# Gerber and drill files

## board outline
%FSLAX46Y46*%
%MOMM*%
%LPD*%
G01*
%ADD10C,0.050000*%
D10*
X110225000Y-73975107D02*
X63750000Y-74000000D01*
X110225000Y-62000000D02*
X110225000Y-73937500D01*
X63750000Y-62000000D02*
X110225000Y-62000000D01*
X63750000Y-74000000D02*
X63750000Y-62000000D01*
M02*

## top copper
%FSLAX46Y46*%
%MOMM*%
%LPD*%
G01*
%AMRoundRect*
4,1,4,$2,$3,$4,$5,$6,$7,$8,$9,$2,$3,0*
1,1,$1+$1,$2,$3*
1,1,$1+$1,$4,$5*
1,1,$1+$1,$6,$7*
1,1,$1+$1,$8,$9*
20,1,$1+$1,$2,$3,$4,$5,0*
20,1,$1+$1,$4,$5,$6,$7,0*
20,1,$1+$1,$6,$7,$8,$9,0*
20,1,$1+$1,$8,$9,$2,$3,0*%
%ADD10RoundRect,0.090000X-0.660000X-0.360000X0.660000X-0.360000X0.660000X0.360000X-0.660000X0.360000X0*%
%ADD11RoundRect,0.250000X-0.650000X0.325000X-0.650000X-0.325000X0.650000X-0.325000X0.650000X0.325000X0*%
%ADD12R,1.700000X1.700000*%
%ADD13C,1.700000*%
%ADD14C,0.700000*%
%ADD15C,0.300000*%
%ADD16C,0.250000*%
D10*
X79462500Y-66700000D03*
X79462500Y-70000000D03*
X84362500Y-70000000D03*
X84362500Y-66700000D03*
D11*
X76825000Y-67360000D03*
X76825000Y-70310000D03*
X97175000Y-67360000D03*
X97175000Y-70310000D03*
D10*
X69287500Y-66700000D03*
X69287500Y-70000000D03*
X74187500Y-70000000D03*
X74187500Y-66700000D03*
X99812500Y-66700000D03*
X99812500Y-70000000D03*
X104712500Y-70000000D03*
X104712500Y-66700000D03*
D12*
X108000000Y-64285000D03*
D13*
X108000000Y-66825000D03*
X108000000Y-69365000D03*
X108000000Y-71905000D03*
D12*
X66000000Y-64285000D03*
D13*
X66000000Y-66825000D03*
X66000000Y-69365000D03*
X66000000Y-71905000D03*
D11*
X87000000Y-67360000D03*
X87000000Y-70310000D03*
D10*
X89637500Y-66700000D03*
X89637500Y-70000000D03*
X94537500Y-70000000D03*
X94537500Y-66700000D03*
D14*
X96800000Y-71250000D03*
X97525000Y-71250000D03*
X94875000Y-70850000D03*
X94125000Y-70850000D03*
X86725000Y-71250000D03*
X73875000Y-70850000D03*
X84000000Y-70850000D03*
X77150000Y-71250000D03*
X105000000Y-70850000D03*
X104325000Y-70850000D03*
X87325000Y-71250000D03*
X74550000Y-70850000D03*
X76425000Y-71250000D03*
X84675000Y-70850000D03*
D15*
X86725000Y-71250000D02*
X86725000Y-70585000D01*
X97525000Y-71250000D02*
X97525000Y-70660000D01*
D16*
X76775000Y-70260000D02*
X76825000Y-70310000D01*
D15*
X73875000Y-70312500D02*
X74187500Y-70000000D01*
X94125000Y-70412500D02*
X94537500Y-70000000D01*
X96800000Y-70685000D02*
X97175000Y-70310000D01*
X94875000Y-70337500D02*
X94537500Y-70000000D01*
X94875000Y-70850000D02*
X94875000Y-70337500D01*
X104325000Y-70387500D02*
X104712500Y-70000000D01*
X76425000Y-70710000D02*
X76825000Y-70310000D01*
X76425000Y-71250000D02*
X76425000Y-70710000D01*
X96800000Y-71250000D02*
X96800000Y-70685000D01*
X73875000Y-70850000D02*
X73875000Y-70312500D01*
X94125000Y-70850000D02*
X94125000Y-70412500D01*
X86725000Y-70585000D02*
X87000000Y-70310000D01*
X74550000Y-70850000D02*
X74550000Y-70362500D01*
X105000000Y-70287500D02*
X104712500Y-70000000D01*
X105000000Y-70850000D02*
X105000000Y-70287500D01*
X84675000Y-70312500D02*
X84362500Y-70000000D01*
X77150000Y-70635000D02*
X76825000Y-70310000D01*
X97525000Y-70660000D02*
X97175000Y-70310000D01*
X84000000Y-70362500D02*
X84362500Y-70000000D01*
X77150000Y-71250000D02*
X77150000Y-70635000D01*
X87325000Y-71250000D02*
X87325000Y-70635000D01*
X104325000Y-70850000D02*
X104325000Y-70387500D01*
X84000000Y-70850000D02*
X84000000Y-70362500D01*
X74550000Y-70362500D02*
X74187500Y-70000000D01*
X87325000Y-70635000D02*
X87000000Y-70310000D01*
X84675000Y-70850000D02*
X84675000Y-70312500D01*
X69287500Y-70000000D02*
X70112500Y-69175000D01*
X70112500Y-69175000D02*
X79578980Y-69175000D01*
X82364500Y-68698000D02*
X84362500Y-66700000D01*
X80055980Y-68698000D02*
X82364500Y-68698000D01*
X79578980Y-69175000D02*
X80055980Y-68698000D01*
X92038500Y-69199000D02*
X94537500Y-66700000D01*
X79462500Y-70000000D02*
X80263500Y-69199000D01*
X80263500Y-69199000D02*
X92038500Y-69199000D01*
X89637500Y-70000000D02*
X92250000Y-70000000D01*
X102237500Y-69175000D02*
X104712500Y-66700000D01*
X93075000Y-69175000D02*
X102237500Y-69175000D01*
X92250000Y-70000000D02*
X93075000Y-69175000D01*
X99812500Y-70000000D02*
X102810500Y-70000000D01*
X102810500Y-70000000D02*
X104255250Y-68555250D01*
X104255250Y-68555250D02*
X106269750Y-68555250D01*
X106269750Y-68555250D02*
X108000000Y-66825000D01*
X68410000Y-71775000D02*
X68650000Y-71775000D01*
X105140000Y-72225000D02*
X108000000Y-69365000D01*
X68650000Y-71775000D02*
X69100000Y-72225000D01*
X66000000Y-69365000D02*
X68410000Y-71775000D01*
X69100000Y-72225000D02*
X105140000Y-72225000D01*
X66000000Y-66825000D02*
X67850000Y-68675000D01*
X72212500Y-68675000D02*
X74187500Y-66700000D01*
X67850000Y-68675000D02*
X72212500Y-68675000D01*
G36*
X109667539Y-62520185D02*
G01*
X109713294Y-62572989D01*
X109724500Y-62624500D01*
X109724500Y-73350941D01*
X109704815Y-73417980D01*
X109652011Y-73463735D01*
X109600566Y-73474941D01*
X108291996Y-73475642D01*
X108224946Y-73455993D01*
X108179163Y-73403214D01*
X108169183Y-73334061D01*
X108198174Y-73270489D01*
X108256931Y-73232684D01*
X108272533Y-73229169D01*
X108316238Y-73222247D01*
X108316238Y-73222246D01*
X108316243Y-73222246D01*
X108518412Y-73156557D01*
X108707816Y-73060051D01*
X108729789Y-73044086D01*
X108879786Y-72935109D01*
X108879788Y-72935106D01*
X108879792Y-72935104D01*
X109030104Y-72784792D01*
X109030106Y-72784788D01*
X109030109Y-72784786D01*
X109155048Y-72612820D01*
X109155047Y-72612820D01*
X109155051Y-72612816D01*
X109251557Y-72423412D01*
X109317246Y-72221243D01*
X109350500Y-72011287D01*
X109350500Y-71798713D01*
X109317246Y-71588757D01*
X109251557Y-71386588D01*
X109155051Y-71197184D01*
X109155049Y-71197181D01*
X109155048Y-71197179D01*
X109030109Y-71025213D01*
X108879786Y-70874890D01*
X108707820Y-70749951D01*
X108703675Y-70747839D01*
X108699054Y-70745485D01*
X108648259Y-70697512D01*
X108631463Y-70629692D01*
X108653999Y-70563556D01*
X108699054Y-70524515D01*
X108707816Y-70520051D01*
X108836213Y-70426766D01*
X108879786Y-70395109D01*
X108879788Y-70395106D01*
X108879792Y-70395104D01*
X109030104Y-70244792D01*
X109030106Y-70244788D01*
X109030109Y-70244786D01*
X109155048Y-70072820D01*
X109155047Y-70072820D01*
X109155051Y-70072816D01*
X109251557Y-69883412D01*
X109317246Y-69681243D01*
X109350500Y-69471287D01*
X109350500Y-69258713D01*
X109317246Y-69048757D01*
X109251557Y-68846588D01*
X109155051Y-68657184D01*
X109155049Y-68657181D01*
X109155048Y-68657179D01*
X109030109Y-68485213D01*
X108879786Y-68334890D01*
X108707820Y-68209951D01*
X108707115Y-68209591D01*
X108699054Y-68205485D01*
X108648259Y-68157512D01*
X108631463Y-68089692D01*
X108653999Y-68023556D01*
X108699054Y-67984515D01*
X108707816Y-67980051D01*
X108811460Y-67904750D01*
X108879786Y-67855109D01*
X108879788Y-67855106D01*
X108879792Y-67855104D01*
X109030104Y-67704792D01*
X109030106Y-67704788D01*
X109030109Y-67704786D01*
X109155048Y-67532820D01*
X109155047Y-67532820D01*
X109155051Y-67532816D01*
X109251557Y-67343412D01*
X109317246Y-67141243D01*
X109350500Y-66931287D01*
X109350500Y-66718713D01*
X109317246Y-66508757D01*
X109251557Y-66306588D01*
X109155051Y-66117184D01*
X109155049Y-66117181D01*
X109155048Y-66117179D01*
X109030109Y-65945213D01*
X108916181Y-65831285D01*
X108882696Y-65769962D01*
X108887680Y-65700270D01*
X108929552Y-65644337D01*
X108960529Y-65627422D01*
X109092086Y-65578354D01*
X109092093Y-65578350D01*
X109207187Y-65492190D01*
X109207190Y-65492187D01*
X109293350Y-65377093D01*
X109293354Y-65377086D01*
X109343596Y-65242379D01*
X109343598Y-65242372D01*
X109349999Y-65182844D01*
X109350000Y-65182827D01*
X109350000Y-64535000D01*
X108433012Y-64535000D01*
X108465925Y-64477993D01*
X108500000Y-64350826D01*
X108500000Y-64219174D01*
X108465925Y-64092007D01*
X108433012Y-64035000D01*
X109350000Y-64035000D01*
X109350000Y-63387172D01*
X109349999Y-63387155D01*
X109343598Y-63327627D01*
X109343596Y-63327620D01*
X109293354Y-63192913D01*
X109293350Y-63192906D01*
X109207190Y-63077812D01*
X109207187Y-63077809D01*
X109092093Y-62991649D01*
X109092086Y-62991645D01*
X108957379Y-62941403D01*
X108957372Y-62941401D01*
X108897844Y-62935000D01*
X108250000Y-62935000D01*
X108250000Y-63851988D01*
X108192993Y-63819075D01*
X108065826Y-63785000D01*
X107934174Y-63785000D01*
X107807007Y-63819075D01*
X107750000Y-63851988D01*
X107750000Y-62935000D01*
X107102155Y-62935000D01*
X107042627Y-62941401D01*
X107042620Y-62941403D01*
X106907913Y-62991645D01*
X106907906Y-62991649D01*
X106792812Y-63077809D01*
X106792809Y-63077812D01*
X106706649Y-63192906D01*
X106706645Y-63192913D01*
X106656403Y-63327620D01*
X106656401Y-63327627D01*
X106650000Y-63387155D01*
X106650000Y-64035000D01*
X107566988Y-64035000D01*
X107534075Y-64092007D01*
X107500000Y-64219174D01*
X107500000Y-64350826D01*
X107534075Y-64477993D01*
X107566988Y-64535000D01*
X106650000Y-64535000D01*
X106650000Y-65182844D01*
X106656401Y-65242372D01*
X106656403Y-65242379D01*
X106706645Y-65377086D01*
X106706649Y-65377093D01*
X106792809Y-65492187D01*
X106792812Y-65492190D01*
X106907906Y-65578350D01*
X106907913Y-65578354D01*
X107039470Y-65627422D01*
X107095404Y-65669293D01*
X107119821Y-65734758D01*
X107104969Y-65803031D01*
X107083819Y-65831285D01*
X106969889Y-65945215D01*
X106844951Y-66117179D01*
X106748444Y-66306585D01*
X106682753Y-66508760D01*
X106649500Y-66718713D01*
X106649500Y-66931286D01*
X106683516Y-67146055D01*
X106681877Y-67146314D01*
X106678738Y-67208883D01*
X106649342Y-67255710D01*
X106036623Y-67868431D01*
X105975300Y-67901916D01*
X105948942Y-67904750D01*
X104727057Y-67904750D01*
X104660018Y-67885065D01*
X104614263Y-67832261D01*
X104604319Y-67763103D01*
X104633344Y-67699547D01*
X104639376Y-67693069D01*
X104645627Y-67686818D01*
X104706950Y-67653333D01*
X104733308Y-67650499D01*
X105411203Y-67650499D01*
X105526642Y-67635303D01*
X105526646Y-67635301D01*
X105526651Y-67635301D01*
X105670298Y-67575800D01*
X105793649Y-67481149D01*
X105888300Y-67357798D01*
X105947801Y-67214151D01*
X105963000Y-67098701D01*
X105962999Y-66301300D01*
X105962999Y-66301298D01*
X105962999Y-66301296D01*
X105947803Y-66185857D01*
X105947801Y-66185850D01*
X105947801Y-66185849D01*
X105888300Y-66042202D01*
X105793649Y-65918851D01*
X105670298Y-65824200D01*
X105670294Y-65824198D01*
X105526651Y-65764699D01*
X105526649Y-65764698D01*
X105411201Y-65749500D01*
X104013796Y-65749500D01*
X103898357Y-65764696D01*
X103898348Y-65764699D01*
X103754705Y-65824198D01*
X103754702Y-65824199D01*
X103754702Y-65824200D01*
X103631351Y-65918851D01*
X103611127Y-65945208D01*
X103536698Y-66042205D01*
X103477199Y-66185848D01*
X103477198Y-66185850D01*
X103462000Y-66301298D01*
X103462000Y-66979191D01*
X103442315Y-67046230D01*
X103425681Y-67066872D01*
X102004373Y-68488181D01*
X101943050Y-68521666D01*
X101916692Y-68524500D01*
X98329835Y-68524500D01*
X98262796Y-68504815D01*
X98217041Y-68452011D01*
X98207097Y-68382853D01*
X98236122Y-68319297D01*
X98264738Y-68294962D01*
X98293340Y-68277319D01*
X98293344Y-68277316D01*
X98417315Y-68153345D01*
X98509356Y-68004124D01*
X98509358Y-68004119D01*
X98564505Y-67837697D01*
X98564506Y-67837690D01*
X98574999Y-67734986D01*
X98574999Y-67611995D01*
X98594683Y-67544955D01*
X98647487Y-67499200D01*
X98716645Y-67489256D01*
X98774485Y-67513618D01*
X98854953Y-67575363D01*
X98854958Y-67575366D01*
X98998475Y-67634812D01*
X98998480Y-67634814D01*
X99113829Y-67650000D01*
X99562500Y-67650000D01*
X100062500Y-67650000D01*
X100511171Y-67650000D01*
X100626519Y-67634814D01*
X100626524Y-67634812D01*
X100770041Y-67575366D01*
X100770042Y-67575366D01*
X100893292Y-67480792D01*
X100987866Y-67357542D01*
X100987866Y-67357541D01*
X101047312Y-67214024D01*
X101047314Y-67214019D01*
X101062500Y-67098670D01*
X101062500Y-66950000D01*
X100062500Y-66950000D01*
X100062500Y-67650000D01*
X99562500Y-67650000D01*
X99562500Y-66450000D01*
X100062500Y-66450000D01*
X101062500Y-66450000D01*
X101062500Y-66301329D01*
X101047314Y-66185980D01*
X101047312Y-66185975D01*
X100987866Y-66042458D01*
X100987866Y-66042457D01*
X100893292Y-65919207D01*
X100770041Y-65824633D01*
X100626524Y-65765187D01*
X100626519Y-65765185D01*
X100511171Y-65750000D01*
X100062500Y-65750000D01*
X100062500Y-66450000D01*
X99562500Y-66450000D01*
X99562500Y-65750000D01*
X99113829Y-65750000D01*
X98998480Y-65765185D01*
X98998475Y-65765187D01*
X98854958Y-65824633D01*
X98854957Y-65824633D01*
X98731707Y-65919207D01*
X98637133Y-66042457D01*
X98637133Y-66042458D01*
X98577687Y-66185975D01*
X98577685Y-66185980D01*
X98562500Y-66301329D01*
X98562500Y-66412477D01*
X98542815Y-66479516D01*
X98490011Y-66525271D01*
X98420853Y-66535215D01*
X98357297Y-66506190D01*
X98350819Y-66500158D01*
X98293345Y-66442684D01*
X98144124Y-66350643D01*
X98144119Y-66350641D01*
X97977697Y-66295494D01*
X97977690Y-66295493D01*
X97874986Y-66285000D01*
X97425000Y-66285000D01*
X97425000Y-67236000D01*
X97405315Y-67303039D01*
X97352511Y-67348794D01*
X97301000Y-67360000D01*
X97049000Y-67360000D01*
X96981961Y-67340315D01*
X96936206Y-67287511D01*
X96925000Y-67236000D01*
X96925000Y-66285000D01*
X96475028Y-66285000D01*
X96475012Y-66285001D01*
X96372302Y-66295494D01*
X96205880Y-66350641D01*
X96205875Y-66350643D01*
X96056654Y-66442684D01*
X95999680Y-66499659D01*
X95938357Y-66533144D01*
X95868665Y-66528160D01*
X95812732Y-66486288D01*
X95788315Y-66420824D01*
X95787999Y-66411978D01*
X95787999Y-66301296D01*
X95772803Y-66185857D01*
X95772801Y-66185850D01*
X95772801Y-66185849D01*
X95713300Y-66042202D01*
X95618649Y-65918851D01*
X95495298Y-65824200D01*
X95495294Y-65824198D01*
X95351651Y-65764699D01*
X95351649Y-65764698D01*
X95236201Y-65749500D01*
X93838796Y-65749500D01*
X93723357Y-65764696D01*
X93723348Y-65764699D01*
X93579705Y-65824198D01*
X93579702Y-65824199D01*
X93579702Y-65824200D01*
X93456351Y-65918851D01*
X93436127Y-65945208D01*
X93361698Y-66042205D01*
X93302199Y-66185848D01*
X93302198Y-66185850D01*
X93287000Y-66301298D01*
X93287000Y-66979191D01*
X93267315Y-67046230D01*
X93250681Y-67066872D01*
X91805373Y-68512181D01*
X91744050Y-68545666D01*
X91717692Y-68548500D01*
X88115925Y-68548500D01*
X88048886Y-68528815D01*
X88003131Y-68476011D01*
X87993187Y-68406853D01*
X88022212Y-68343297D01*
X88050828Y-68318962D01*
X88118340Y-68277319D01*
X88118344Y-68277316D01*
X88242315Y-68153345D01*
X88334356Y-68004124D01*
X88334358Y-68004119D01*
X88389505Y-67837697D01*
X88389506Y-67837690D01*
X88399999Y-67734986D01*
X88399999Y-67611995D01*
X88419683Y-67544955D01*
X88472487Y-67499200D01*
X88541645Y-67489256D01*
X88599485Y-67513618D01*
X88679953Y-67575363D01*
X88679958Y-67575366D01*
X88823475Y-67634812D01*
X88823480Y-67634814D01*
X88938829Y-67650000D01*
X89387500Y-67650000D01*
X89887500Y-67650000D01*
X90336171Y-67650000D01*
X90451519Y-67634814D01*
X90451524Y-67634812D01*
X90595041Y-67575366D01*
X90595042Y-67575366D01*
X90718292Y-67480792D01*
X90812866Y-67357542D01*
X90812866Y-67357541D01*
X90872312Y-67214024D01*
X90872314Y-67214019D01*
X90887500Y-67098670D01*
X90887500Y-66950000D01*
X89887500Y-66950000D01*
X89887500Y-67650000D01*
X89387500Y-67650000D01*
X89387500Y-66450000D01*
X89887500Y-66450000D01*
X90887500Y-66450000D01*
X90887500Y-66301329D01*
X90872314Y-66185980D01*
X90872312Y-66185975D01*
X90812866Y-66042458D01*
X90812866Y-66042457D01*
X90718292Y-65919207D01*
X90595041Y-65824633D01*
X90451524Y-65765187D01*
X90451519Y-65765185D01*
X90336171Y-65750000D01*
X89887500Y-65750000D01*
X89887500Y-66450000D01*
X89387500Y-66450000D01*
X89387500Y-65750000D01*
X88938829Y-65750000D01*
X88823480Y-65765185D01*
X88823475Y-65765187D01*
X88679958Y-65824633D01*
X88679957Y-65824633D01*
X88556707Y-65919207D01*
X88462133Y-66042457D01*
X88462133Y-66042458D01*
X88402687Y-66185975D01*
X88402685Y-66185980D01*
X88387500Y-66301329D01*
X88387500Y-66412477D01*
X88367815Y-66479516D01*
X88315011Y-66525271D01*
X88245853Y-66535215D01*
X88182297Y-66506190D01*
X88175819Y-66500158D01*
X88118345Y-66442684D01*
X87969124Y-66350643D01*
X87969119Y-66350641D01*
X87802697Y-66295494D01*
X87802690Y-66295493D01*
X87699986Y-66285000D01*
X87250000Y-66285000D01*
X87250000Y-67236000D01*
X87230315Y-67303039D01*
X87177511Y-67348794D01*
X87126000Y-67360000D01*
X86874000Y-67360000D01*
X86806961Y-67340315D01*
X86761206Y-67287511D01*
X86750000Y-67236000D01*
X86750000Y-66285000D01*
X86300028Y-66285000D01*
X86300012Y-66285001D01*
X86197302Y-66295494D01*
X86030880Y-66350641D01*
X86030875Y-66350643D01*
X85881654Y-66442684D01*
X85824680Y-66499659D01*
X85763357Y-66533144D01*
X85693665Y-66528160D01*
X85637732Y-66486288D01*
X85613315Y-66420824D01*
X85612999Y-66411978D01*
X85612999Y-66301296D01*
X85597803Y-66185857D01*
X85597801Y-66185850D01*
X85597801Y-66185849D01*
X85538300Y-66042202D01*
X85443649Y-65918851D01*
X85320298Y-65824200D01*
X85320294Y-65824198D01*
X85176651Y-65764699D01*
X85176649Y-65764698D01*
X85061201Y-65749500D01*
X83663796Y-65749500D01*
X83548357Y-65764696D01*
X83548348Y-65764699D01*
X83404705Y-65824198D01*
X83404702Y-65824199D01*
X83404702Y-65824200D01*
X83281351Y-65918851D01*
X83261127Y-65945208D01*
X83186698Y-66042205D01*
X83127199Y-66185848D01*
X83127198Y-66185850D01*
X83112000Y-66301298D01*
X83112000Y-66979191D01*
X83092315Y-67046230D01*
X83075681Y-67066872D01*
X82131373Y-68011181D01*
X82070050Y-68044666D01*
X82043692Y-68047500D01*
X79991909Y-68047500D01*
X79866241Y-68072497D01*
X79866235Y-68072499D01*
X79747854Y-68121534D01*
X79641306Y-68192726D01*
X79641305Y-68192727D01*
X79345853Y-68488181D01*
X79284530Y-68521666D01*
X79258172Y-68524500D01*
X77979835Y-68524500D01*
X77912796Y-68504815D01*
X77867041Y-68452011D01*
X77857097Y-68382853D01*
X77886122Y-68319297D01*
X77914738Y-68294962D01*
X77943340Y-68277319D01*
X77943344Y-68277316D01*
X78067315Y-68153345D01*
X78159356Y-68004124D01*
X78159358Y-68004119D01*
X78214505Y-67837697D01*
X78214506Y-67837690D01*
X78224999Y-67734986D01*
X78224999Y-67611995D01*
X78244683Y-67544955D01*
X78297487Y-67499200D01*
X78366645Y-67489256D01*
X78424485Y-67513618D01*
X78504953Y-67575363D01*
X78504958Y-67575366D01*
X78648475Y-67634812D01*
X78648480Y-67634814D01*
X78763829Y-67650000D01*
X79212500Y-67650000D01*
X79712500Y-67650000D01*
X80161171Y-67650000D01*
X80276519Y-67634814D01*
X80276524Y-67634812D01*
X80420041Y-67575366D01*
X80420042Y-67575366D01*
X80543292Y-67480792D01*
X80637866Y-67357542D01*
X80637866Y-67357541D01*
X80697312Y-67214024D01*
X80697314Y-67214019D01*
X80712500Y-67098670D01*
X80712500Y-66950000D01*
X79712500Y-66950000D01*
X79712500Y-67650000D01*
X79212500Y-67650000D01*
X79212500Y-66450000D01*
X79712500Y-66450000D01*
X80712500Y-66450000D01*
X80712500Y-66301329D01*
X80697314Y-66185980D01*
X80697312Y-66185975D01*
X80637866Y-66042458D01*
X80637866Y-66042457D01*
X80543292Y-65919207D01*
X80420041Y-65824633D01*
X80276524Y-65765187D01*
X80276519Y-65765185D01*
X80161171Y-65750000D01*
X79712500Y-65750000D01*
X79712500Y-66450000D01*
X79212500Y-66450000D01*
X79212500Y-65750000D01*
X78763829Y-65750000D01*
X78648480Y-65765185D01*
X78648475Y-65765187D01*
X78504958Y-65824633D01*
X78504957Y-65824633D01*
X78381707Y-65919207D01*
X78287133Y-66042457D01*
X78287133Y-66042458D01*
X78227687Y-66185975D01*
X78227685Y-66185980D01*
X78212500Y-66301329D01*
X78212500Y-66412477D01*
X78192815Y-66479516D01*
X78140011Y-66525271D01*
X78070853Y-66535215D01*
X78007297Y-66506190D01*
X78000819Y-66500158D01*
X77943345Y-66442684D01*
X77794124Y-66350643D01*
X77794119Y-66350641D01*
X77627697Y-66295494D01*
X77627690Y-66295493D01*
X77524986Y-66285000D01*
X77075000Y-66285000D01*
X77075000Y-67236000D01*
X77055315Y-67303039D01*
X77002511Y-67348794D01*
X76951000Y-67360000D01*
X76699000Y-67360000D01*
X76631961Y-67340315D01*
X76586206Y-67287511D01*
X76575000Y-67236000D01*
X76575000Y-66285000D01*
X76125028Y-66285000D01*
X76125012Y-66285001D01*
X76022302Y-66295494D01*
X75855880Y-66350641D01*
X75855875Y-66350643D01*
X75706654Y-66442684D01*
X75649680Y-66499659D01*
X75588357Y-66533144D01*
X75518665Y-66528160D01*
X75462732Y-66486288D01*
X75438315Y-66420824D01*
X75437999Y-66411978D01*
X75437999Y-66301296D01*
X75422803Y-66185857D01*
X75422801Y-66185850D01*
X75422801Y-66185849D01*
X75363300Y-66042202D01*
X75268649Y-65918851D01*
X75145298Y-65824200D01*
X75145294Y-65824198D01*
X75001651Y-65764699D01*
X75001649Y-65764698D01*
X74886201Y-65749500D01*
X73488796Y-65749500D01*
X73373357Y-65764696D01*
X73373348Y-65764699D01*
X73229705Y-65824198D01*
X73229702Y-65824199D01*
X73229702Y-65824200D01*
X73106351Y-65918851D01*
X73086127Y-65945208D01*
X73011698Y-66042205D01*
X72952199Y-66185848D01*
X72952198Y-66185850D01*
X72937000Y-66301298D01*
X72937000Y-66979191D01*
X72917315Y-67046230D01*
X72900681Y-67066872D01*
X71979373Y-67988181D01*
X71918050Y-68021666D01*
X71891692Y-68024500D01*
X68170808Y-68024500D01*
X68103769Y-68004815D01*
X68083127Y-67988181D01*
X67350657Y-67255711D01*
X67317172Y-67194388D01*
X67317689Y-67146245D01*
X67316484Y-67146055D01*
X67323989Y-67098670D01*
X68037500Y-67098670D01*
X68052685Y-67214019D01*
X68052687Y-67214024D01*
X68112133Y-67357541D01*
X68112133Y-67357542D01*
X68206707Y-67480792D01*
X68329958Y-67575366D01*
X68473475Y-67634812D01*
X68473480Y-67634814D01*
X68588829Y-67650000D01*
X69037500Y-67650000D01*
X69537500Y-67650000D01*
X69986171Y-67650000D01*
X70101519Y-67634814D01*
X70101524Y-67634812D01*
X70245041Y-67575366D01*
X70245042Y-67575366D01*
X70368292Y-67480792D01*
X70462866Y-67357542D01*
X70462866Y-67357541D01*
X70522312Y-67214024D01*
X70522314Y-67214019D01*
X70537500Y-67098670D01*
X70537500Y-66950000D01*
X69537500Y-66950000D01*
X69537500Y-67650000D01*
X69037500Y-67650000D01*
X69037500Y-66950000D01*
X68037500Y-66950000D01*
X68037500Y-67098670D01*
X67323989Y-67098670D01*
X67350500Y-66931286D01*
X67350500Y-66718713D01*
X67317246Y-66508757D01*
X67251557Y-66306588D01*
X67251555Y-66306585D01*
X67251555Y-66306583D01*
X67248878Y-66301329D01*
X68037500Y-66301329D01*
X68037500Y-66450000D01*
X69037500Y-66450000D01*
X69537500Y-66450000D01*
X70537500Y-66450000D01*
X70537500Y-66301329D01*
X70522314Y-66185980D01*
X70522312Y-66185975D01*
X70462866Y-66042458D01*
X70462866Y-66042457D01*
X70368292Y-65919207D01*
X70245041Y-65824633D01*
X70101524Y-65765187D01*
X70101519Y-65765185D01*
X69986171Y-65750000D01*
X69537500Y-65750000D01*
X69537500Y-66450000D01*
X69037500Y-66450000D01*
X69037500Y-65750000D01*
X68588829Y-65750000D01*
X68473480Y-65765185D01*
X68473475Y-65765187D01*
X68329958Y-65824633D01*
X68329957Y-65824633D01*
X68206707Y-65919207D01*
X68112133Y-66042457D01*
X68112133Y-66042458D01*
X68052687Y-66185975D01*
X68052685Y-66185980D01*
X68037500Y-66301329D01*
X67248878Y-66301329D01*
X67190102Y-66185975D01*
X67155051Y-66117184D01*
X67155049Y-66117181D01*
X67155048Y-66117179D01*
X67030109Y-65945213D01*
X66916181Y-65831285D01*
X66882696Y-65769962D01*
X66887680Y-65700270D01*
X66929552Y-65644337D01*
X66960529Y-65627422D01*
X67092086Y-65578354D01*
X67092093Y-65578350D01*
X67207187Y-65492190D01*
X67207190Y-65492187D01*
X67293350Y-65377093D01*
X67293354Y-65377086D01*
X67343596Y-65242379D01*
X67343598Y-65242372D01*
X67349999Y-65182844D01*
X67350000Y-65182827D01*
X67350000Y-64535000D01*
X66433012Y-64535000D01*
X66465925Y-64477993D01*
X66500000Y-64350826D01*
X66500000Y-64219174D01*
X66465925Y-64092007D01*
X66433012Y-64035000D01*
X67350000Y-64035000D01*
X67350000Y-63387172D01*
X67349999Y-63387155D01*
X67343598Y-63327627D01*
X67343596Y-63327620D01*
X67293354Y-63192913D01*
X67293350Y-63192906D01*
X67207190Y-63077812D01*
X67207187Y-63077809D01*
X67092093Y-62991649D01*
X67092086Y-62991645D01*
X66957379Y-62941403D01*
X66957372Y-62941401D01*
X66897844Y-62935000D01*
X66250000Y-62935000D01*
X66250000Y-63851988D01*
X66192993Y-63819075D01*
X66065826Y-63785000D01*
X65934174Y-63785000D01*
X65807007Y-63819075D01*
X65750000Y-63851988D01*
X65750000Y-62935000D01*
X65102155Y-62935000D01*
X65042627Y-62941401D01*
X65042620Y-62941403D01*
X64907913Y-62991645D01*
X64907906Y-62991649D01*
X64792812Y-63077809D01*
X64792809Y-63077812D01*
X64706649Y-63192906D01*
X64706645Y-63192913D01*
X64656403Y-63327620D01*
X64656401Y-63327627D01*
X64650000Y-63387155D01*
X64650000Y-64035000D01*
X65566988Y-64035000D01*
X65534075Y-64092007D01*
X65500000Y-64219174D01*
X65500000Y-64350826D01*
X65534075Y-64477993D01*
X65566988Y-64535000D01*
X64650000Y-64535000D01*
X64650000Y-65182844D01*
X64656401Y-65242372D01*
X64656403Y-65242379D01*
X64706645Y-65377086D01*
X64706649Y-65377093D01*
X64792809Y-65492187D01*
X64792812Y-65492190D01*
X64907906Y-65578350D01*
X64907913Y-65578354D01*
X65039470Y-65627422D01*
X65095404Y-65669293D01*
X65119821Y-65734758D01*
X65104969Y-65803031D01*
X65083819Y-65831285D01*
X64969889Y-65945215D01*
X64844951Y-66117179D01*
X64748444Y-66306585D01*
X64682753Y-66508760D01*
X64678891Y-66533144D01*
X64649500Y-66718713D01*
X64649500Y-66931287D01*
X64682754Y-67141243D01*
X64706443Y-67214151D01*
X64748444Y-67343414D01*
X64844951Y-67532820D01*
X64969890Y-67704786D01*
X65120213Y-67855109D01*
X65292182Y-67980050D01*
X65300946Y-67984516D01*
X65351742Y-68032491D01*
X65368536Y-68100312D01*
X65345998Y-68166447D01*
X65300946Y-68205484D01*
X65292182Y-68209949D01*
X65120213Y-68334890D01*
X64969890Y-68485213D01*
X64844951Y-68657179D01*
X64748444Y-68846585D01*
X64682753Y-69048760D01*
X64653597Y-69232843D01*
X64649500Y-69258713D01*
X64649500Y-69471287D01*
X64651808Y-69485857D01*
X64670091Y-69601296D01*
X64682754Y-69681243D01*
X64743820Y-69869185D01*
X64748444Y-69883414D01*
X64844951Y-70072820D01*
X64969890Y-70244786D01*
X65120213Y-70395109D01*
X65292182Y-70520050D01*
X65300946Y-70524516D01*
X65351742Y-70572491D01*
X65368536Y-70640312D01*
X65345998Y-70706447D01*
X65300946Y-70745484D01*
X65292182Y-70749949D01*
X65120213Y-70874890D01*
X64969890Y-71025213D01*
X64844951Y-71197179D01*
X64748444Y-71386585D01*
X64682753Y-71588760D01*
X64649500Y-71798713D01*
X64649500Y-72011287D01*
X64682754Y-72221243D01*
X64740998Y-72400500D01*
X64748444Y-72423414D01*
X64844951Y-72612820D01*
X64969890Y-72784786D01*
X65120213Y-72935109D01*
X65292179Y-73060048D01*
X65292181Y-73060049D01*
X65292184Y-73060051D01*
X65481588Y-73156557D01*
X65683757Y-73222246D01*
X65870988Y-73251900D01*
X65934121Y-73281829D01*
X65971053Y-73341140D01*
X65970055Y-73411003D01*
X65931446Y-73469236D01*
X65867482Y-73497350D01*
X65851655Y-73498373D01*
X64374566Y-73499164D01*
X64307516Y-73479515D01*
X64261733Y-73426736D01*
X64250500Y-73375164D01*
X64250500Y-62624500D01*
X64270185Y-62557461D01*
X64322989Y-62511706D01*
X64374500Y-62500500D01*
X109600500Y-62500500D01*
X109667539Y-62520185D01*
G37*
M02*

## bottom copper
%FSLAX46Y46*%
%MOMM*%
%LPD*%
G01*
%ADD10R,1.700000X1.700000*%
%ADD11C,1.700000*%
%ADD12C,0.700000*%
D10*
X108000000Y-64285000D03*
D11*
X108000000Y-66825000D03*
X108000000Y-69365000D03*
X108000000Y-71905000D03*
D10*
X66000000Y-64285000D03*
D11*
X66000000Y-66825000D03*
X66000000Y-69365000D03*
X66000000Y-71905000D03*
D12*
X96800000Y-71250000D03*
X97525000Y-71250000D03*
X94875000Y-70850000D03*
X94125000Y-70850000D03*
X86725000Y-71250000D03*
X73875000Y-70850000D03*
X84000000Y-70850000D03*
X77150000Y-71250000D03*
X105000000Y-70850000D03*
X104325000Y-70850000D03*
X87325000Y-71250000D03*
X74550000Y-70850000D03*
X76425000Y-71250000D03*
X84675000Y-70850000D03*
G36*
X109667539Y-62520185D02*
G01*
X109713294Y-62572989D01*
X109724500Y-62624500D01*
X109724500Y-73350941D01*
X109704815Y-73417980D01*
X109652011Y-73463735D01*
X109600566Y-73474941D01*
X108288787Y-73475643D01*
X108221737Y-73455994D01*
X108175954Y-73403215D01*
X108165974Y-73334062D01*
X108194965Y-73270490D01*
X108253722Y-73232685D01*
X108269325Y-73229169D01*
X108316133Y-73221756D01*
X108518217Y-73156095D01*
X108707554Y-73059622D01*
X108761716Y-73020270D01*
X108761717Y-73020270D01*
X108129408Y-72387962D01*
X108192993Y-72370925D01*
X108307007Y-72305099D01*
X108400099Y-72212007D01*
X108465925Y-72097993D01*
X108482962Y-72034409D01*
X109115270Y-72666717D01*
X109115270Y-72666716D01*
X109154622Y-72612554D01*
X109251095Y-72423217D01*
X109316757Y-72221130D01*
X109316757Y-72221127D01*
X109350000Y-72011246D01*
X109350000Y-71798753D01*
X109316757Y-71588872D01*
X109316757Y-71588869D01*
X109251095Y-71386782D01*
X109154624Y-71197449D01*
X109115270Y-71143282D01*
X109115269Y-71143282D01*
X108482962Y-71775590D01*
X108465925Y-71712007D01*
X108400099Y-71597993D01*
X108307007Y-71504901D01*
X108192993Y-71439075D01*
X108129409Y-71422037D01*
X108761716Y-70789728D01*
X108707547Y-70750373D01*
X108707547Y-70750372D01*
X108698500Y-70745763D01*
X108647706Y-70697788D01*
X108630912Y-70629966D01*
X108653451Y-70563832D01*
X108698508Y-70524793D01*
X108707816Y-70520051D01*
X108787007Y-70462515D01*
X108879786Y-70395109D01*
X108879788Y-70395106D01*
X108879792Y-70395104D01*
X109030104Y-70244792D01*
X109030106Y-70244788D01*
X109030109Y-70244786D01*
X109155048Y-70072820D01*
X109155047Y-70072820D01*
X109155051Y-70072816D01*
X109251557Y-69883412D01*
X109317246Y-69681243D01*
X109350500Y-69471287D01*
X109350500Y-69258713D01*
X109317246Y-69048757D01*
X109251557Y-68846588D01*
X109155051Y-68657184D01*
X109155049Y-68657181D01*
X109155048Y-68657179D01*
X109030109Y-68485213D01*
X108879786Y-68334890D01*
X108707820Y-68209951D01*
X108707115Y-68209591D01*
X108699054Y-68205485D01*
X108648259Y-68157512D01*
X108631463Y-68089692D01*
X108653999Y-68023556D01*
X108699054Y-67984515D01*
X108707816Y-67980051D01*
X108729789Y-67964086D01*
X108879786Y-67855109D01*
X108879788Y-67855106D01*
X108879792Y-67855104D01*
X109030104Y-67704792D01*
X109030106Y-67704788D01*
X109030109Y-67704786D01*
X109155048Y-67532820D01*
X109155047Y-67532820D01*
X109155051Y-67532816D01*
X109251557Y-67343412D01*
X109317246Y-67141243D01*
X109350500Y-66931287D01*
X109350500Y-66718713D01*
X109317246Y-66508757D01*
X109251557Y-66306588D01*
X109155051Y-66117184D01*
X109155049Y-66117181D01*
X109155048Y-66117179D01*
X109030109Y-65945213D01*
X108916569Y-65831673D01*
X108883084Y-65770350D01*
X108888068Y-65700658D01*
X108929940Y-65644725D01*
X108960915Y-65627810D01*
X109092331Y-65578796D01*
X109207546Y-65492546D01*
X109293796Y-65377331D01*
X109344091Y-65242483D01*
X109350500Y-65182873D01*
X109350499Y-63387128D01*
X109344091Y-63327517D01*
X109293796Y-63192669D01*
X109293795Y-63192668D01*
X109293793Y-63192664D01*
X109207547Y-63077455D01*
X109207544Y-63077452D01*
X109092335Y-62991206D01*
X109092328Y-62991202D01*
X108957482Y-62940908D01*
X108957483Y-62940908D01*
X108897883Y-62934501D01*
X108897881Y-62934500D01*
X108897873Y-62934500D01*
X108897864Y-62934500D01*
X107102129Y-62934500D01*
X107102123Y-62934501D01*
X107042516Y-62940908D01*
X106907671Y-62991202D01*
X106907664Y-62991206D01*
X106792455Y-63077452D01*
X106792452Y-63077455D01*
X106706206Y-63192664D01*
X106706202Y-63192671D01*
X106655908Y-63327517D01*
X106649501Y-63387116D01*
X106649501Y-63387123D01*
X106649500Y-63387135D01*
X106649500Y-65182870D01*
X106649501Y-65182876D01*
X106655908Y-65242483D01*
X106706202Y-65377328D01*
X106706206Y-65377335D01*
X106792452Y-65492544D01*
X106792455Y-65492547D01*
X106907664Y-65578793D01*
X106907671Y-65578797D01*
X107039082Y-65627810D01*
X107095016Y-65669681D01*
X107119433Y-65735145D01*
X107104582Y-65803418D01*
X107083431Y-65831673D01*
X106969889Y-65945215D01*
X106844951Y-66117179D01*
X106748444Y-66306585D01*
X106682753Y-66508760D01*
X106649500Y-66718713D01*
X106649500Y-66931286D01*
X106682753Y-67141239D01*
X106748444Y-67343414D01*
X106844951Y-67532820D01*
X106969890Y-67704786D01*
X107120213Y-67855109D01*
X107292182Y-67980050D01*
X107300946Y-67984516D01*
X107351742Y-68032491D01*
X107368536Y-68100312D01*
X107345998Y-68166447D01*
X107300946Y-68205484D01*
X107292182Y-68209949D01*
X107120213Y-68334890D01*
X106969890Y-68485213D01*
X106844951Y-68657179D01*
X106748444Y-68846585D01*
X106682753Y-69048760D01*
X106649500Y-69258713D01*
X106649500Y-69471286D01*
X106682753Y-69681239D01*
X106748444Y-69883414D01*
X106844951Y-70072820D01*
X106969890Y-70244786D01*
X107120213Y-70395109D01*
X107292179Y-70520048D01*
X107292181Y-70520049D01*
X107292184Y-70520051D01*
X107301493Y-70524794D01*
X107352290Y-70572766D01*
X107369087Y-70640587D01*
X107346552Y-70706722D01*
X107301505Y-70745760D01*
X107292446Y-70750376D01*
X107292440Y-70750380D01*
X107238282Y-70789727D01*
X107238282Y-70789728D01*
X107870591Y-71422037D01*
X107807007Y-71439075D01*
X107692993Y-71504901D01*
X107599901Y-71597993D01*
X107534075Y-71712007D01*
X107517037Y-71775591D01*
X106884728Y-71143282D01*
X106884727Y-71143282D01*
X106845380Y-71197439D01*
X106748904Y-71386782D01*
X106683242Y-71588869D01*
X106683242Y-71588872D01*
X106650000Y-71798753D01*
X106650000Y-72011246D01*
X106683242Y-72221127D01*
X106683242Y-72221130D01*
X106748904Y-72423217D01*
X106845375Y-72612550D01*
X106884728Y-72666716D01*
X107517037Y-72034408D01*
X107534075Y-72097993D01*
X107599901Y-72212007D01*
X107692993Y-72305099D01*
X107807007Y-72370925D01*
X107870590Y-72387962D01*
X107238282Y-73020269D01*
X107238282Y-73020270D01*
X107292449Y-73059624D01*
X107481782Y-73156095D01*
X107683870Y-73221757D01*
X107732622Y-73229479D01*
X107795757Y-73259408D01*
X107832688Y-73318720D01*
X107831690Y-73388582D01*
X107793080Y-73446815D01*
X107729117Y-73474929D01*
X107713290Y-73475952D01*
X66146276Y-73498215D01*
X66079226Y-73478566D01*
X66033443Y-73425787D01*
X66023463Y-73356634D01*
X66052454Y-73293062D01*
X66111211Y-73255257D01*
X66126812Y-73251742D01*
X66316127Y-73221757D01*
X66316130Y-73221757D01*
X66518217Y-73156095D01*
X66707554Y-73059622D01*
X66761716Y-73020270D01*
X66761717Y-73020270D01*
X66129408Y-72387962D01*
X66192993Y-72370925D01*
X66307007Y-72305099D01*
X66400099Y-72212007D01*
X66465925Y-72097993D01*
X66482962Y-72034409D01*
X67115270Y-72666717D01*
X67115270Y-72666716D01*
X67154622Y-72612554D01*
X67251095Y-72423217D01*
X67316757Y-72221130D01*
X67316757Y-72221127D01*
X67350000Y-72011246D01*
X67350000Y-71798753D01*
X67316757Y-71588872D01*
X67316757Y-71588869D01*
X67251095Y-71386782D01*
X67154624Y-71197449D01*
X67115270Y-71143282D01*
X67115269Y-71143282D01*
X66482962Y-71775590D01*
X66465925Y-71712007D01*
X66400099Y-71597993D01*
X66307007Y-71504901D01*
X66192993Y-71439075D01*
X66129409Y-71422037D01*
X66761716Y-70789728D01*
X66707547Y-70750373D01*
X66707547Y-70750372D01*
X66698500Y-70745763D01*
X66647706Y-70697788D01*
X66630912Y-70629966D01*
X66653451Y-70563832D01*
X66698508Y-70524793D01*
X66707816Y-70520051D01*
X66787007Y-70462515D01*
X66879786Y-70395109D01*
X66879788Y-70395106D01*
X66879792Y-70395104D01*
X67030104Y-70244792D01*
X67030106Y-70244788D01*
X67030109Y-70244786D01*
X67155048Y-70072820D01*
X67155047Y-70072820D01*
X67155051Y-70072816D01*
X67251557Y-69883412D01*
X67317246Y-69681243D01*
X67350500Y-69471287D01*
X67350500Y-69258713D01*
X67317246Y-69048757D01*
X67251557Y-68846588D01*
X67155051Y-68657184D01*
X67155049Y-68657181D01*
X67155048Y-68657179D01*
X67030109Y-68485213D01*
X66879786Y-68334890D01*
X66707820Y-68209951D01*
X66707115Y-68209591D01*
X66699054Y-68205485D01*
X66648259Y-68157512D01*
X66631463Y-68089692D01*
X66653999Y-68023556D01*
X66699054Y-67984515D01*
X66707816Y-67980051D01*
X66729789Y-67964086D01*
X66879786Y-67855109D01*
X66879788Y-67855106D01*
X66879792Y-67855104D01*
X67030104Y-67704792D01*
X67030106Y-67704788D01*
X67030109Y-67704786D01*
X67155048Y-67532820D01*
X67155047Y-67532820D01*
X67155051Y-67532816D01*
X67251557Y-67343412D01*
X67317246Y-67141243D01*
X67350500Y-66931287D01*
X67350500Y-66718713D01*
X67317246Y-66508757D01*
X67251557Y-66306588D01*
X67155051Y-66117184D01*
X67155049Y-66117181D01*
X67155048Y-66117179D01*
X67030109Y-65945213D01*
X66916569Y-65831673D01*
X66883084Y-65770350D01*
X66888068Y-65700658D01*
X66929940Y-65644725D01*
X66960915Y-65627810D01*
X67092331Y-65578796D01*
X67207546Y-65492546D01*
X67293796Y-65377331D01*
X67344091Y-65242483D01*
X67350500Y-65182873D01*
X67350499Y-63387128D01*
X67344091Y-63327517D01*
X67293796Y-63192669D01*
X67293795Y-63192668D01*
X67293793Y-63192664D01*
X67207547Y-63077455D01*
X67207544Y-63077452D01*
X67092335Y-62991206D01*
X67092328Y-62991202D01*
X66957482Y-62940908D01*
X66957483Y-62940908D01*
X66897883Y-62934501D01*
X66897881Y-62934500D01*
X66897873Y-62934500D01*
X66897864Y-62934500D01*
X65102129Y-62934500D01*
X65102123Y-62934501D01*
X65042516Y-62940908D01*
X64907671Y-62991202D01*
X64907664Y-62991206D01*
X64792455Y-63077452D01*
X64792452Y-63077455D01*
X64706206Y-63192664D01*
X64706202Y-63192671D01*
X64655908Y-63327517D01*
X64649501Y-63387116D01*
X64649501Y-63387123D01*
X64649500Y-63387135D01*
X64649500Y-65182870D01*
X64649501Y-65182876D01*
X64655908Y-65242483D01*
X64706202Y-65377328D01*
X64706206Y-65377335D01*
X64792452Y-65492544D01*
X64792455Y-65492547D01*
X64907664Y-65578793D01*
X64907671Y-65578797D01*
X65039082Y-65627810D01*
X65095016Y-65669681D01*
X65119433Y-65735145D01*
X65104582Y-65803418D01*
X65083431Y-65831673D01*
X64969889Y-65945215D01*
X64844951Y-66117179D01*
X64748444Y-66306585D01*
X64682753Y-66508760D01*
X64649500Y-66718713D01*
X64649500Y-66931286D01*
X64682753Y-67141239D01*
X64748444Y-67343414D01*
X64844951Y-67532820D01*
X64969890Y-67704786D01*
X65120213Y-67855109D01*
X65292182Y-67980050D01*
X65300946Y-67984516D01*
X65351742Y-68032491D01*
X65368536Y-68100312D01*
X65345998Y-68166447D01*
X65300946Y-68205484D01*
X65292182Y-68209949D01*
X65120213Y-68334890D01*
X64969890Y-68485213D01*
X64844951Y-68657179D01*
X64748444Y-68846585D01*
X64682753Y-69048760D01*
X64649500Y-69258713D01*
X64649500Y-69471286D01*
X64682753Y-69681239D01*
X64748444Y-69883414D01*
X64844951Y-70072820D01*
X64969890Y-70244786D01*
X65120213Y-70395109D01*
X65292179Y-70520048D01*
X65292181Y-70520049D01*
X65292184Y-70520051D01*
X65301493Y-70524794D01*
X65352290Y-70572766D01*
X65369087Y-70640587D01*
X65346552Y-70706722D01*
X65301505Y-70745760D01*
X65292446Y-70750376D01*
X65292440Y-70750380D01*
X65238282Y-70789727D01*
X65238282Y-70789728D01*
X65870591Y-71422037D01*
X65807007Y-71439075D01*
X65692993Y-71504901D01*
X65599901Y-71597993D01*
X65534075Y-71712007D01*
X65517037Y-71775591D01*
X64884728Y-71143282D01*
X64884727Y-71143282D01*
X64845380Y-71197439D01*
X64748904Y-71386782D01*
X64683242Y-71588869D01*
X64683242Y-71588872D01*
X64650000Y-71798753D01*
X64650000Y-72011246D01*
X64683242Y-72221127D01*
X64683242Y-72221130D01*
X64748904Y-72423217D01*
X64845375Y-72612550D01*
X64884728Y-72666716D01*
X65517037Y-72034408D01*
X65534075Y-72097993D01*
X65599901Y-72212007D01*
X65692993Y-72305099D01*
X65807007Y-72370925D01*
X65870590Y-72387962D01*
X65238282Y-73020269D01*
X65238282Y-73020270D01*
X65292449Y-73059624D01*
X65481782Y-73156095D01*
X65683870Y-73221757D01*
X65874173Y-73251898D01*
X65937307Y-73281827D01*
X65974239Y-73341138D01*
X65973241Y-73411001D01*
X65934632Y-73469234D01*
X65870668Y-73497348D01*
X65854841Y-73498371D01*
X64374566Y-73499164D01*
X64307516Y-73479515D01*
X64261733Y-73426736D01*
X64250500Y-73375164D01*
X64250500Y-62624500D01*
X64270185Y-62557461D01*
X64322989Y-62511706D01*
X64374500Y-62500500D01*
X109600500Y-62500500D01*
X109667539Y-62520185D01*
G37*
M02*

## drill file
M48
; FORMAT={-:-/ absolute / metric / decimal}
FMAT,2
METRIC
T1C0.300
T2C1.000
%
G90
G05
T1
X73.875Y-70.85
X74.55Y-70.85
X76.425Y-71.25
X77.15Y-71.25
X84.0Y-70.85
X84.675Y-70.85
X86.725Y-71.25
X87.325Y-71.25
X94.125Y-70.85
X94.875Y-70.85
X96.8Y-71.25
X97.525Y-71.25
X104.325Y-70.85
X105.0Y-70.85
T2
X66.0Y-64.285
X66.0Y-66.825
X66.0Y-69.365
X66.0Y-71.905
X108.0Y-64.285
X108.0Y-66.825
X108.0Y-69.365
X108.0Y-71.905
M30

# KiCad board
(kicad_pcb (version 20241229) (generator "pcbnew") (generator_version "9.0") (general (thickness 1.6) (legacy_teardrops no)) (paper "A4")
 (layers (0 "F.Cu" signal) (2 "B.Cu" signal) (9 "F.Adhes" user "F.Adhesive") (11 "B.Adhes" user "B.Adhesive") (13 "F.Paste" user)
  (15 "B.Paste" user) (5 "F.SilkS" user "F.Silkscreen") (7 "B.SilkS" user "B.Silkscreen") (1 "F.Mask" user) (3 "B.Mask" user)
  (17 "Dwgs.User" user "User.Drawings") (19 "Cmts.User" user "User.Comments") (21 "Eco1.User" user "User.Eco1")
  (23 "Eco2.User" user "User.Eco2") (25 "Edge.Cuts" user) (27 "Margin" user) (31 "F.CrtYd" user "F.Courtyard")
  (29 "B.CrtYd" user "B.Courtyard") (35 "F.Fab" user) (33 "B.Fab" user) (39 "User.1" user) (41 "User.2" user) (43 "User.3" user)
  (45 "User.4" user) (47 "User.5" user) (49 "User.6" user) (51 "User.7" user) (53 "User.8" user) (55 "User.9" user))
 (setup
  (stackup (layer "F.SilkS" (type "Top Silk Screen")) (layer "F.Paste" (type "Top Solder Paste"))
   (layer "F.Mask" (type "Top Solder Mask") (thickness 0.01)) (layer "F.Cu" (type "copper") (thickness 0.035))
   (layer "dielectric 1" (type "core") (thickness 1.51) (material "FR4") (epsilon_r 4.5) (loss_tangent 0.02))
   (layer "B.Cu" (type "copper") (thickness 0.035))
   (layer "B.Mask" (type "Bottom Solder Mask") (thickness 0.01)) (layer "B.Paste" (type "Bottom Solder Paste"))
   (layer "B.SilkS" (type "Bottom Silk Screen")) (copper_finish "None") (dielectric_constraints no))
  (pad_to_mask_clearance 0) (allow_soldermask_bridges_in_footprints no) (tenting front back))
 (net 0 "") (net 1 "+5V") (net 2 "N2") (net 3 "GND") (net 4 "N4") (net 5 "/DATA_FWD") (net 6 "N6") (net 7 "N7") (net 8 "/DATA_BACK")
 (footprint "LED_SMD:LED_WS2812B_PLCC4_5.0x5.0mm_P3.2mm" (layer "F.Cu") (at 81.9125 68.35)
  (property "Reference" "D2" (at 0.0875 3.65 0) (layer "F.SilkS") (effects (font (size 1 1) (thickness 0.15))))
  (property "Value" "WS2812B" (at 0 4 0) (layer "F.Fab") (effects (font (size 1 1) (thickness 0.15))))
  (pad "1" smd roundrect (at -2.45 -1.65) (size 1.5 0.9) (layers "F.Cu" "F.Mask" "F.Paste") (roundrect_rratio 0.1) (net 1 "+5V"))
  (pad "2" smd roundrect (at -2.45 1.65) (size 1.5 0.9) (layers "F.Cu" "F.Mask" "F.Paste") (roundrect_rratio 0.1) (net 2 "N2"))
  (pad "3" smd roundrect (at 2.45 1.65) (size 1.5 0.9) (layers "F.Cu" "F.Mask" "F.Paste") (roundrect_rratio 0.1) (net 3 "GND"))
  (pad "4" smd roundrect (at 2.45 -1.65) (size 1.5 0.9) (layers "F.Cu" "F.Mask" "F.Paste") (roundrect_rratio 0.1) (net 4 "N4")))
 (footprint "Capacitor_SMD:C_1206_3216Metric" (layer "F.Cu") (at 76.825 68.835 -90)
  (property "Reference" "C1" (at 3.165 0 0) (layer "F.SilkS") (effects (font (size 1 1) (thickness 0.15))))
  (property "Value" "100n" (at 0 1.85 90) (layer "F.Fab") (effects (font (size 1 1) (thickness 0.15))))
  (pad "1" smd roundrect (at -1.475 0 270) (size 1.15 1.8) (layers "F.Cu" "F.Mask" "F.Paste") (roundrect_rratio 0.217391) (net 1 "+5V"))
  (pad "2" smd roundrect (at 1.475 0 270) (size 1.15 1.8) (layers "F.Cu" "F.Mask" "F.Paste") (roundrect_rratio 0.217391) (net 3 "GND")))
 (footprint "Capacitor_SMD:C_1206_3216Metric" (layer "F.Cu") (at 97.175 68.835 -90)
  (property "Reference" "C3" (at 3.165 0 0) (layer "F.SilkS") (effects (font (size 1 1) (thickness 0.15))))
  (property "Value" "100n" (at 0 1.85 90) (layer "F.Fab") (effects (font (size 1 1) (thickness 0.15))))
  (pad "1" smd roundrect (at -1.475 0 270) (size 1.15 1.8) (layers "F.Cu" "F.Mask" "F.Paste") (roundrect_rratio 0.217391) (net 1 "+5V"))
  (pad "2" smd roundrect (at 1.475 0 270) (size 1.15 1.8) (layers "F.Cu" "F.Mask" "F.Paste") (roundrect_rratio 0.217391) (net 3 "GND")))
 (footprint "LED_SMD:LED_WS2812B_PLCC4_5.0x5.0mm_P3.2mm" (layer "F.Cu") (at 71.7375 68.35)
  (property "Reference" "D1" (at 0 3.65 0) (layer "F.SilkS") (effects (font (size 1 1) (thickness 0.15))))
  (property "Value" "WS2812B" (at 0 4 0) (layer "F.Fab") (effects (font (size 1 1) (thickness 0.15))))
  (pad "1" smd roundrect (at -2.45 -1.65) (size 1.5 0.9) (layers "F.Cu" "F.Mask" "F.Paste") (roundrect_rratio 0.1) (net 1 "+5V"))
  (pad "2" smd roundrect (at -2.45 1.65) (size 1.5 0.9) (layers "F.Cu" "F.Mask" "F.Paste") (roundrect_rratio 0.1) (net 4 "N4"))
  (pad "3" smd roundrect (at 2.45 1.65) (size 1.5 0.9) (layers "F.Cu" "F.Mask" "F.Paste") (roundrect_rratio 0.1) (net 3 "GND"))
  (pad "4" smd roundrect (at 2.45 -1.65) (size 1.5 0.9) (layers "F.Cu" "F.Mask" "F.Paste") (roundrect_rratio 0.1) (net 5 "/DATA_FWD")))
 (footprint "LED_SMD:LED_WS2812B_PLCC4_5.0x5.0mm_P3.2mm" (layer "F.Cu") (at 102.2625 68.35)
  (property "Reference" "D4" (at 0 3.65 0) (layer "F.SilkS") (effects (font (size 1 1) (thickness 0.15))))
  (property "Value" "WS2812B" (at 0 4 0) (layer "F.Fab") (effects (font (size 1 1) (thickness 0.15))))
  (pad "1" smd roundrect (at -2.45 -1.65) (size 1.5 0.9) (layers "F.Cu" "F.Mask" "F.Paste") (roundrect_rratio 0.1) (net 1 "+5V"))
  (pad "2" smd roundrect (at -2.45 1.65) (size 1.5 0.9) (layers "F.Cu" "F.Mask" "F.Paste") (roundrect_rratio 0.1) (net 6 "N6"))
  (pad "3" smd roundrect (at 2.45 1.65) (size 1.5 0.9) (layers "F.Cu" "F.Mask" "F.Paste") (roundrect_rratio 0.1) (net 3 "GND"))
  (pad "4" smd roundrect (at 2.45 -1.65) (size 1.5 0.9) (layers "F.Cu" "F.Mask" "F.Paste") (roundrect_rratio 0.1) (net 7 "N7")))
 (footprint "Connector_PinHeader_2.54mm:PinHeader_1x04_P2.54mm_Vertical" (layer "F.Cu") (at 108 64.285)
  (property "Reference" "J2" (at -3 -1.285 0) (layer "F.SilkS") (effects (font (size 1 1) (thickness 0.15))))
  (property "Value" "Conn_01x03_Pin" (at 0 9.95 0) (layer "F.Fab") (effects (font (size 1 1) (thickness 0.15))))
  (pad "1" thru_hole rect (at 0 0) (size 1.7 1.7) (drill 1) (layers "*.Cu" "*.Mask") (remove_unused_layers no) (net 1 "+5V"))
  (pad "2" thru_hole circle (at 0 2.54) (size 1.7 1.7) (drill 1) (layers "*.Cu" "*.Mask") (remove_unused_layers no) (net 6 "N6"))
  (pad "3" thru_hole circle (at 0 5.08) (size 1.7 1.7) (drill 1) (layers "*.Cu" "*.Mask") (remove_unused_layers no) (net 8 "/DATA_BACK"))
  (pad "4" thru_hole circle (at 0 7.62) (size 1.7 1.7) (drill 1) (layers "*.Cu" "*.Mask") (remove_unused_layers no) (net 3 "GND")))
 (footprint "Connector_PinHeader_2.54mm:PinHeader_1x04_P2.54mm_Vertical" (layer "F.Cu") (at 66 64.285)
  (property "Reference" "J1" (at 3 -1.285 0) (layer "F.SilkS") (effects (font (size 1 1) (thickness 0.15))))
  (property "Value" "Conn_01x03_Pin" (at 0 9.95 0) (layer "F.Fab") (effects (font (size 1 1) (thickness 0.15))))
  (pad "1" thru_hole rect (at 0 0) (size 1.7 1.7) (drill 1) (layers "*.Cu" "*.Mask") (remove_unused_layers no) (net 1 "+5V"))
  (pad "2" thru_hole circle (at 0 2.54) (size 1.7 1.7) (drill 1) (layers "*.Cu" "*.Mask") (remove_unused_layers no) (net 5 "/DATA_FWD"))
  (pad "3" thru_hole circle (at 0 5.08) (size 1.7 1.7) (drill 1) (layers "*.Cu" "*.Mask") (remove_unused_layers no) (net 8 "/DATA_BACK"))
  (pad "4" thru_hole circle (at 0 7.62) (size 1.7 1.7) (drill 1) (layers "*.Cu" "*.Mask") (remove_unused_layers no) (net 3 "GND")))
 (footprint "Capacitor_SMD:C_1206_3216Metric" (layer "F.Cu") (at 87 68.835 -90)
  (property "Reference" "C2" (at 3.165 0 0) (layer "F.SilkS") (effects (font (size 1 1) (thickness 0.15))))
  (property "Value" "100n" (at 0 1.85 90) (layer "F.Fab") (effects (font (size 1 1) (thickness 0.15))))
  (pad "1" smd roundrect (at -1.475 0 270) (size 1.15 1.8) (layers "F.Cu" "F.Mask" "F.Paste") (roundrect_rratio 0.217391) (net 1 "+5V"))
  (pad "2" smd roundrect (at 1.475 0 270) (size 1.15 1.8) (layers "F.Cu" "F.Mask" "F.Paste") (roundrect_rratio 0.217391) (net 3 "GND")))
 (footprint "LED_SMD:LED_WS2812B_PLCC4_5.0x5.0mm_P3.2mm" (layer "F.Cu") (at 92.0875 68.35)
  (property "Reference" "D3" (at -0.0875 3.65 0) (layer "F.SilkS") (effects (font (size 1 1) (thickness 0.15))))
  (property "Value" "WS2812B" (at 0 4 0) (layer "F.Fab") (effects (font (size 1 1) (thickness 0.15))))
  (pad "1" smd roundrect (at -2.45 -1.65) (size 1.5 0.9) (layers "F.Cu" "F.Mask" "F.Paste") (roundrect_rratio 0.1) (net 1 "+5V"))
  (pad "2" smd roundrect (at -2.45 1.65) (size 1.5 0.9) (layers "F.Cu" "F.Mask" "F.Paste") (roundrect_rratio 0.1) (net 7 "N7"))
  (pad "3" smd roundrect (at 2.45 1.65) (size 1.5 0.9) (layers "F.Cu" "F.Mask" "F.Paste") (roundrect_rratio 0.1) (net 3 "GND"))
  (pad "4" smd roundrect (at 2.45 -1.65) (size 1.5 0.9) (layers "F.Cu" "F.Mask" "F.Paste") (roundrect_rratio 0.1) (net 2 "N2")))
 (gr_line (start 110.225 73.975107) (end 63.75 74) (stroke (width 0.05) (type default)) (layer "Edge.Cuts"))
 (gr_line (start 110.225 62) (end 110.225 73.9375) (stroke (width 0.05) (type default)) (layer "Edge.Cuts"))
 (gr_line (start 63.75 62) (end 110.225 62) (stroke (width 0.05) (type default)) (layer "Edge.Cuts"))
 (gr_line (start 63.75 74) (end 63.75 62) (stroke (width 0.05) (type default)) (layer "Edge.Cuts"))
 (segment (start 86.725 71.25) (end 86.725 70.585) (width 0.3) (layer "F.Cu") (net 3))
 (segment (start 97.525 71.25) (end 97.525 70.66) (width 0.3) (layer "F.Cu") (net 3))
 (segment (start 76.775 70.26) (end 76.825 70.31) (width 0.25) (layer "F.Cu") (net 3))
 (segment (start 73.875 70.3125) (end 74.1875 70) (width 0.3) (layer "F.Cu") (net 3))
 (segment (start 94.125 70.4125) (end 94.5375 70) (width 0.3) (layer "F.Cu") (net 3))
 (segment (start 96.8 70.685) (end 97.175 70.31) (width 0.3) (layer "F.Cu") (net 3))
 (segment (start 94.875 70.3375) (end 94.5375 70) (width 0.3) (layer "F.Cu") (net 3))
 (segment (start 94.875 70.85) (end 94.875 70.3375) (width 0.3) (layer "F.Cu") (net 3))
 (segment (start 104.325 70.3875) (end 104.7125 70) (width 0.3) (layer "F.Cu") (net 3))
 (segment (start 76.425 70.71) (end 76.825 70.31) (width 0.3) (layer "F.Cu") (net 3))
 (segment (start 76.425 71.25) (end 76.425 70.71) (width 0.3) (layer "F.Cu") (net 3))
 (segment (start 96.8 71.25) (end 96.8 70.685) (width 0.3) (layer "F.Cu") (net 3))
 (segment (start 73.875 70.85) (end 73.875 70.3125) (width 0.3) (layer "F.Cu") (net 3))
 (segment (start 94.125 70.85) (end 94.125 70.4125) (width 0.3) (layer "F.Cu") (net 3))
 (segment (start 86.725 70.585) (end 87 70.31) (width 0.3) (layer "F.Cu") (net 3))
 (segment (start 74.55 70.85) (end 74.55 70.3625) (width 0.3) (layer "F.Cu") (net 3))
 (segment (start 105 70.2875) (end 104.7125 70) (width 0.3) (layer "F.Cu") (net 3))
 (segment (start 105 70.85) (end 105 70.2875) (width 0.3) (layer "F.Cu") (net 3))
 (segment (start 84.675 70.3125) (end 84.3625 70) (width 0.3) (layer "F.Cu") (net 3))
 (segment (start 77.15 70.635) (end 76.825 70.31) (width 0.3) (layer "F.Cu") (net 3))
 (segment (start 97.525 70.66) (end 97.175 70.31) (width 0.3) (layer "F.Cu") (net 3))
 (segment (start 84 70.3625) (end 84.3625 70) (width 0.3) (layer "F.Cu") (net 3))
 (segment (start 77.15 71.25) (end 77.15 70.635) (width 0.3) (layer "F.Cu") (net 3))
 (segment (start 87.325 71.25) (end 87.325 70.635) (width 0.3) (layer "F.Cu") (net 3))
 (segment (start 104.325 70.85) (end 104.325 70.3875) (width 0.3) (layer "F.Cu") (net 3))
 (segment (start 84 70.85) (end 84 70.3625) (width 0.3) (layer "F.Cu") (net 3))
 (segment (start 74.55 70.3625) (end 74.1875 70) (width 0.3) (layer "F.Cu") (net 3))
 (segment (start 87.325 70.635) (end 87 70.31) (width 0.3) (layer "F.Cu") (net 3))
 (segment (start 84.675 70.85) (end 84.675 70.3125) (width 0.3) (layer "F.Cu") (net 3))
 (via (at 96.8 71.25) (size 0.7) (drill 0.3) (layers "F.Cu" "B.Cu") (free yes) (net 3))
 (via (at 97.525 71.25) (size 0.7) (drill 0.3) (layers "F.Cu" "B.Cu") (free yes) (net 3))
 (via (at 94.875 70.85) (size 0.7) (drill 0.3) (layers "F.Cu" "B.Cu") (free yes) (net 3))
 (via (at 94.125 70.85) (size 0.7) (drill 0.3) (layers "F.Cu" "B.Cu") (free yes) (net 3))
 (via (at 86.725 71.25) (size 0.7) (drill 0.3) (layers "F.Cu" "B.Cu") (free yes) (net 3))
 (via (at 73.875 70.85) (size 0.7) (drill 0.3) (layers "F.Cu" "B.Cu") (free yes) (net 3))
 (via (at 84 70.85) (size 0.7) (drill 0.3) (layers "F.Cu" "B.Cu") (free yes) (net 3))
 (via (at 77.15 71.25) (size 0.7) (drill 0.3) (layers "F.Cu" "B.Cu") (free yes) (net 3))
 (via (at 105 70.85) (size 0.7) (drill 0.3) (layers "F.Cu" "B.Cu") (free yes) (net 3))
 (via (at 104.325 70.85) (size 0.7) (drill 0.3) (layers "F.Cu" "B.Cu") (free yes) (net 3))
 (via (at 87.325 71.25) (size 0.7) (drill 0.3) (layers "F.Cu" "B.Cu") (free yes) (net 3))
 (via (at 74.55 70.85) (size 0.7) (drill 0.3) (layers "F.Cu" "B.Cu") (free yes) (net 3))
 (via (at 76.425 71.25) (size 0.7) (drill 0.3) (layers "F.Cu" "B.Cu") (free yes) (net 3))
 (via (at 84.675 70.85) (size 0.7) (drill 0.3) (layers "F.Cu" "B.Cu") (free yes) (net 3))
 (segment (start 69.2875 70) (end 70.1125 69.175) (width 0.3) (layer "F.Cu") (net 4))
 (segment (start 70.1125 69.175) (end 79.57898 69.175) (width 0.3) (layer "F.Cu") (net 4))
 (segment (start 82.3645 68.698) (end 84.3625 66.7) (width 0.3) (layer "F.Cu") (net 4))
 (segment (start 80.05598 68.698) (end 82.3645 68.698) (width 0.3) (layer "F.Cu") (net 4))
 (segment (start 79.57898 69.175) (end 80.05598 68.698) (width 0.3) (layer "F.Cu") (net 4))
 (segment (start 92.0385 69.199) (end 94.5375 66.7) (width 0.3) (layer "F.Cu") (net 2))
 (segment (start 79.4625 70) (end 80.2635 69.199) (width 0.3) (layer "F.Cu") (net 2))
 (segment (start 80.2635 69.199) (end 92.0385 69.199) (width 0.3) (layer "F.Cu") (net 2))
 (segment (start 89.6375 70) (end 92.25 70) (width 0.3) (layer "F.Cu") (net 7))
 (segment (start 102.2375 69.175) (end 104.7125 66.7) (width 0.3) (layer "F.Cu") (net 7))
 (segment (start 93.075 69.175) (end 102.2375 69.175) (width 0.3) (layer "F.Cu") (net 7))
 (segment (start 92.25 70) (end 93.075 69.175) (width 0.3) (layer "F.Cu") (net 7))
 (segment (start 99.8125 70) (end 102.8105 70) (width 0.3) (layer "F.Cu") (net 6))
 (segment (start 102.8105 70) (end 104.25525 68.55525) (width 0.3) (layer "F.Cu") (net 6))
 (segment (start 104.25525 68.55525) (end 106.26975 68.55525) (width 0.3) (layer "F.Cu") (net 6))
 (segment (start 106.26975 68.55525) (end 108 66.825) (width 0.3) (layer "F.Cu") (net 6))
 (segment (start 68.41 71.775) (end 68.65 71.775) (width 0.3) (layer "F.Cu") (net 8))
 (segment (start 105.14 72.225) (end 108 69.365) (width 0.3) (layer "F.Cu") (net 8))
 (segment (start 68.65 71.775) (end 69.1 72.225) (width 0.3) (layer "F.Cu") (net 8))
 (segment (start 66 69.365) (end 68.41 71.775) (width 0.3) (layer "F.Cu") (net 8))
 (segment (start 69.1 72.225) (end 105.14 72.225) (width 0.3) (layer "F.Cu") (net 8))
 (segment (start 66 66.825) (end 67.85 68.675) (width 0.3) (layer "F.Cu") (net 5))
 (segment (start 72.2125 68.675) (end 74.1875 66.7) (width 0.3) (layer "F.Cu") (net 5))
 (segment (start 67.85 68.675) (end 72.2125 68.675) (width 0.3) (layer "F.Cu") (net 5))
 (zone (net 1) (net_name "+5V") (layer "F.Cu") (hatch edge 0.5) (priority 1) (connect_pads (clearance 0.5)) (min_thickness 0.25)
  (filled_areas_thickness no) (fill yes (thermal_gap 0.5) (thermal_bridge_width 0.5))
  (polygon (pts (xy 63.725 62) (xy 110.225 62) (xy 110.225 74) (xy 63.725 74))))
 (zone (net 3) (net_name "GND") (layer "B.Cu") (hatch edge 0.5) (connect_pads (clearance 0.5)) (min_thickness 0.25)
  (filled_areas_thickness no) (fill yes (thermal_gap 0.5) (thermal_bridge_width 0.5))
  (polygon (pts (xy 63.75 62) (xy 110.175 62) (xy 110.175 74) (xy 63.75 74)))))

